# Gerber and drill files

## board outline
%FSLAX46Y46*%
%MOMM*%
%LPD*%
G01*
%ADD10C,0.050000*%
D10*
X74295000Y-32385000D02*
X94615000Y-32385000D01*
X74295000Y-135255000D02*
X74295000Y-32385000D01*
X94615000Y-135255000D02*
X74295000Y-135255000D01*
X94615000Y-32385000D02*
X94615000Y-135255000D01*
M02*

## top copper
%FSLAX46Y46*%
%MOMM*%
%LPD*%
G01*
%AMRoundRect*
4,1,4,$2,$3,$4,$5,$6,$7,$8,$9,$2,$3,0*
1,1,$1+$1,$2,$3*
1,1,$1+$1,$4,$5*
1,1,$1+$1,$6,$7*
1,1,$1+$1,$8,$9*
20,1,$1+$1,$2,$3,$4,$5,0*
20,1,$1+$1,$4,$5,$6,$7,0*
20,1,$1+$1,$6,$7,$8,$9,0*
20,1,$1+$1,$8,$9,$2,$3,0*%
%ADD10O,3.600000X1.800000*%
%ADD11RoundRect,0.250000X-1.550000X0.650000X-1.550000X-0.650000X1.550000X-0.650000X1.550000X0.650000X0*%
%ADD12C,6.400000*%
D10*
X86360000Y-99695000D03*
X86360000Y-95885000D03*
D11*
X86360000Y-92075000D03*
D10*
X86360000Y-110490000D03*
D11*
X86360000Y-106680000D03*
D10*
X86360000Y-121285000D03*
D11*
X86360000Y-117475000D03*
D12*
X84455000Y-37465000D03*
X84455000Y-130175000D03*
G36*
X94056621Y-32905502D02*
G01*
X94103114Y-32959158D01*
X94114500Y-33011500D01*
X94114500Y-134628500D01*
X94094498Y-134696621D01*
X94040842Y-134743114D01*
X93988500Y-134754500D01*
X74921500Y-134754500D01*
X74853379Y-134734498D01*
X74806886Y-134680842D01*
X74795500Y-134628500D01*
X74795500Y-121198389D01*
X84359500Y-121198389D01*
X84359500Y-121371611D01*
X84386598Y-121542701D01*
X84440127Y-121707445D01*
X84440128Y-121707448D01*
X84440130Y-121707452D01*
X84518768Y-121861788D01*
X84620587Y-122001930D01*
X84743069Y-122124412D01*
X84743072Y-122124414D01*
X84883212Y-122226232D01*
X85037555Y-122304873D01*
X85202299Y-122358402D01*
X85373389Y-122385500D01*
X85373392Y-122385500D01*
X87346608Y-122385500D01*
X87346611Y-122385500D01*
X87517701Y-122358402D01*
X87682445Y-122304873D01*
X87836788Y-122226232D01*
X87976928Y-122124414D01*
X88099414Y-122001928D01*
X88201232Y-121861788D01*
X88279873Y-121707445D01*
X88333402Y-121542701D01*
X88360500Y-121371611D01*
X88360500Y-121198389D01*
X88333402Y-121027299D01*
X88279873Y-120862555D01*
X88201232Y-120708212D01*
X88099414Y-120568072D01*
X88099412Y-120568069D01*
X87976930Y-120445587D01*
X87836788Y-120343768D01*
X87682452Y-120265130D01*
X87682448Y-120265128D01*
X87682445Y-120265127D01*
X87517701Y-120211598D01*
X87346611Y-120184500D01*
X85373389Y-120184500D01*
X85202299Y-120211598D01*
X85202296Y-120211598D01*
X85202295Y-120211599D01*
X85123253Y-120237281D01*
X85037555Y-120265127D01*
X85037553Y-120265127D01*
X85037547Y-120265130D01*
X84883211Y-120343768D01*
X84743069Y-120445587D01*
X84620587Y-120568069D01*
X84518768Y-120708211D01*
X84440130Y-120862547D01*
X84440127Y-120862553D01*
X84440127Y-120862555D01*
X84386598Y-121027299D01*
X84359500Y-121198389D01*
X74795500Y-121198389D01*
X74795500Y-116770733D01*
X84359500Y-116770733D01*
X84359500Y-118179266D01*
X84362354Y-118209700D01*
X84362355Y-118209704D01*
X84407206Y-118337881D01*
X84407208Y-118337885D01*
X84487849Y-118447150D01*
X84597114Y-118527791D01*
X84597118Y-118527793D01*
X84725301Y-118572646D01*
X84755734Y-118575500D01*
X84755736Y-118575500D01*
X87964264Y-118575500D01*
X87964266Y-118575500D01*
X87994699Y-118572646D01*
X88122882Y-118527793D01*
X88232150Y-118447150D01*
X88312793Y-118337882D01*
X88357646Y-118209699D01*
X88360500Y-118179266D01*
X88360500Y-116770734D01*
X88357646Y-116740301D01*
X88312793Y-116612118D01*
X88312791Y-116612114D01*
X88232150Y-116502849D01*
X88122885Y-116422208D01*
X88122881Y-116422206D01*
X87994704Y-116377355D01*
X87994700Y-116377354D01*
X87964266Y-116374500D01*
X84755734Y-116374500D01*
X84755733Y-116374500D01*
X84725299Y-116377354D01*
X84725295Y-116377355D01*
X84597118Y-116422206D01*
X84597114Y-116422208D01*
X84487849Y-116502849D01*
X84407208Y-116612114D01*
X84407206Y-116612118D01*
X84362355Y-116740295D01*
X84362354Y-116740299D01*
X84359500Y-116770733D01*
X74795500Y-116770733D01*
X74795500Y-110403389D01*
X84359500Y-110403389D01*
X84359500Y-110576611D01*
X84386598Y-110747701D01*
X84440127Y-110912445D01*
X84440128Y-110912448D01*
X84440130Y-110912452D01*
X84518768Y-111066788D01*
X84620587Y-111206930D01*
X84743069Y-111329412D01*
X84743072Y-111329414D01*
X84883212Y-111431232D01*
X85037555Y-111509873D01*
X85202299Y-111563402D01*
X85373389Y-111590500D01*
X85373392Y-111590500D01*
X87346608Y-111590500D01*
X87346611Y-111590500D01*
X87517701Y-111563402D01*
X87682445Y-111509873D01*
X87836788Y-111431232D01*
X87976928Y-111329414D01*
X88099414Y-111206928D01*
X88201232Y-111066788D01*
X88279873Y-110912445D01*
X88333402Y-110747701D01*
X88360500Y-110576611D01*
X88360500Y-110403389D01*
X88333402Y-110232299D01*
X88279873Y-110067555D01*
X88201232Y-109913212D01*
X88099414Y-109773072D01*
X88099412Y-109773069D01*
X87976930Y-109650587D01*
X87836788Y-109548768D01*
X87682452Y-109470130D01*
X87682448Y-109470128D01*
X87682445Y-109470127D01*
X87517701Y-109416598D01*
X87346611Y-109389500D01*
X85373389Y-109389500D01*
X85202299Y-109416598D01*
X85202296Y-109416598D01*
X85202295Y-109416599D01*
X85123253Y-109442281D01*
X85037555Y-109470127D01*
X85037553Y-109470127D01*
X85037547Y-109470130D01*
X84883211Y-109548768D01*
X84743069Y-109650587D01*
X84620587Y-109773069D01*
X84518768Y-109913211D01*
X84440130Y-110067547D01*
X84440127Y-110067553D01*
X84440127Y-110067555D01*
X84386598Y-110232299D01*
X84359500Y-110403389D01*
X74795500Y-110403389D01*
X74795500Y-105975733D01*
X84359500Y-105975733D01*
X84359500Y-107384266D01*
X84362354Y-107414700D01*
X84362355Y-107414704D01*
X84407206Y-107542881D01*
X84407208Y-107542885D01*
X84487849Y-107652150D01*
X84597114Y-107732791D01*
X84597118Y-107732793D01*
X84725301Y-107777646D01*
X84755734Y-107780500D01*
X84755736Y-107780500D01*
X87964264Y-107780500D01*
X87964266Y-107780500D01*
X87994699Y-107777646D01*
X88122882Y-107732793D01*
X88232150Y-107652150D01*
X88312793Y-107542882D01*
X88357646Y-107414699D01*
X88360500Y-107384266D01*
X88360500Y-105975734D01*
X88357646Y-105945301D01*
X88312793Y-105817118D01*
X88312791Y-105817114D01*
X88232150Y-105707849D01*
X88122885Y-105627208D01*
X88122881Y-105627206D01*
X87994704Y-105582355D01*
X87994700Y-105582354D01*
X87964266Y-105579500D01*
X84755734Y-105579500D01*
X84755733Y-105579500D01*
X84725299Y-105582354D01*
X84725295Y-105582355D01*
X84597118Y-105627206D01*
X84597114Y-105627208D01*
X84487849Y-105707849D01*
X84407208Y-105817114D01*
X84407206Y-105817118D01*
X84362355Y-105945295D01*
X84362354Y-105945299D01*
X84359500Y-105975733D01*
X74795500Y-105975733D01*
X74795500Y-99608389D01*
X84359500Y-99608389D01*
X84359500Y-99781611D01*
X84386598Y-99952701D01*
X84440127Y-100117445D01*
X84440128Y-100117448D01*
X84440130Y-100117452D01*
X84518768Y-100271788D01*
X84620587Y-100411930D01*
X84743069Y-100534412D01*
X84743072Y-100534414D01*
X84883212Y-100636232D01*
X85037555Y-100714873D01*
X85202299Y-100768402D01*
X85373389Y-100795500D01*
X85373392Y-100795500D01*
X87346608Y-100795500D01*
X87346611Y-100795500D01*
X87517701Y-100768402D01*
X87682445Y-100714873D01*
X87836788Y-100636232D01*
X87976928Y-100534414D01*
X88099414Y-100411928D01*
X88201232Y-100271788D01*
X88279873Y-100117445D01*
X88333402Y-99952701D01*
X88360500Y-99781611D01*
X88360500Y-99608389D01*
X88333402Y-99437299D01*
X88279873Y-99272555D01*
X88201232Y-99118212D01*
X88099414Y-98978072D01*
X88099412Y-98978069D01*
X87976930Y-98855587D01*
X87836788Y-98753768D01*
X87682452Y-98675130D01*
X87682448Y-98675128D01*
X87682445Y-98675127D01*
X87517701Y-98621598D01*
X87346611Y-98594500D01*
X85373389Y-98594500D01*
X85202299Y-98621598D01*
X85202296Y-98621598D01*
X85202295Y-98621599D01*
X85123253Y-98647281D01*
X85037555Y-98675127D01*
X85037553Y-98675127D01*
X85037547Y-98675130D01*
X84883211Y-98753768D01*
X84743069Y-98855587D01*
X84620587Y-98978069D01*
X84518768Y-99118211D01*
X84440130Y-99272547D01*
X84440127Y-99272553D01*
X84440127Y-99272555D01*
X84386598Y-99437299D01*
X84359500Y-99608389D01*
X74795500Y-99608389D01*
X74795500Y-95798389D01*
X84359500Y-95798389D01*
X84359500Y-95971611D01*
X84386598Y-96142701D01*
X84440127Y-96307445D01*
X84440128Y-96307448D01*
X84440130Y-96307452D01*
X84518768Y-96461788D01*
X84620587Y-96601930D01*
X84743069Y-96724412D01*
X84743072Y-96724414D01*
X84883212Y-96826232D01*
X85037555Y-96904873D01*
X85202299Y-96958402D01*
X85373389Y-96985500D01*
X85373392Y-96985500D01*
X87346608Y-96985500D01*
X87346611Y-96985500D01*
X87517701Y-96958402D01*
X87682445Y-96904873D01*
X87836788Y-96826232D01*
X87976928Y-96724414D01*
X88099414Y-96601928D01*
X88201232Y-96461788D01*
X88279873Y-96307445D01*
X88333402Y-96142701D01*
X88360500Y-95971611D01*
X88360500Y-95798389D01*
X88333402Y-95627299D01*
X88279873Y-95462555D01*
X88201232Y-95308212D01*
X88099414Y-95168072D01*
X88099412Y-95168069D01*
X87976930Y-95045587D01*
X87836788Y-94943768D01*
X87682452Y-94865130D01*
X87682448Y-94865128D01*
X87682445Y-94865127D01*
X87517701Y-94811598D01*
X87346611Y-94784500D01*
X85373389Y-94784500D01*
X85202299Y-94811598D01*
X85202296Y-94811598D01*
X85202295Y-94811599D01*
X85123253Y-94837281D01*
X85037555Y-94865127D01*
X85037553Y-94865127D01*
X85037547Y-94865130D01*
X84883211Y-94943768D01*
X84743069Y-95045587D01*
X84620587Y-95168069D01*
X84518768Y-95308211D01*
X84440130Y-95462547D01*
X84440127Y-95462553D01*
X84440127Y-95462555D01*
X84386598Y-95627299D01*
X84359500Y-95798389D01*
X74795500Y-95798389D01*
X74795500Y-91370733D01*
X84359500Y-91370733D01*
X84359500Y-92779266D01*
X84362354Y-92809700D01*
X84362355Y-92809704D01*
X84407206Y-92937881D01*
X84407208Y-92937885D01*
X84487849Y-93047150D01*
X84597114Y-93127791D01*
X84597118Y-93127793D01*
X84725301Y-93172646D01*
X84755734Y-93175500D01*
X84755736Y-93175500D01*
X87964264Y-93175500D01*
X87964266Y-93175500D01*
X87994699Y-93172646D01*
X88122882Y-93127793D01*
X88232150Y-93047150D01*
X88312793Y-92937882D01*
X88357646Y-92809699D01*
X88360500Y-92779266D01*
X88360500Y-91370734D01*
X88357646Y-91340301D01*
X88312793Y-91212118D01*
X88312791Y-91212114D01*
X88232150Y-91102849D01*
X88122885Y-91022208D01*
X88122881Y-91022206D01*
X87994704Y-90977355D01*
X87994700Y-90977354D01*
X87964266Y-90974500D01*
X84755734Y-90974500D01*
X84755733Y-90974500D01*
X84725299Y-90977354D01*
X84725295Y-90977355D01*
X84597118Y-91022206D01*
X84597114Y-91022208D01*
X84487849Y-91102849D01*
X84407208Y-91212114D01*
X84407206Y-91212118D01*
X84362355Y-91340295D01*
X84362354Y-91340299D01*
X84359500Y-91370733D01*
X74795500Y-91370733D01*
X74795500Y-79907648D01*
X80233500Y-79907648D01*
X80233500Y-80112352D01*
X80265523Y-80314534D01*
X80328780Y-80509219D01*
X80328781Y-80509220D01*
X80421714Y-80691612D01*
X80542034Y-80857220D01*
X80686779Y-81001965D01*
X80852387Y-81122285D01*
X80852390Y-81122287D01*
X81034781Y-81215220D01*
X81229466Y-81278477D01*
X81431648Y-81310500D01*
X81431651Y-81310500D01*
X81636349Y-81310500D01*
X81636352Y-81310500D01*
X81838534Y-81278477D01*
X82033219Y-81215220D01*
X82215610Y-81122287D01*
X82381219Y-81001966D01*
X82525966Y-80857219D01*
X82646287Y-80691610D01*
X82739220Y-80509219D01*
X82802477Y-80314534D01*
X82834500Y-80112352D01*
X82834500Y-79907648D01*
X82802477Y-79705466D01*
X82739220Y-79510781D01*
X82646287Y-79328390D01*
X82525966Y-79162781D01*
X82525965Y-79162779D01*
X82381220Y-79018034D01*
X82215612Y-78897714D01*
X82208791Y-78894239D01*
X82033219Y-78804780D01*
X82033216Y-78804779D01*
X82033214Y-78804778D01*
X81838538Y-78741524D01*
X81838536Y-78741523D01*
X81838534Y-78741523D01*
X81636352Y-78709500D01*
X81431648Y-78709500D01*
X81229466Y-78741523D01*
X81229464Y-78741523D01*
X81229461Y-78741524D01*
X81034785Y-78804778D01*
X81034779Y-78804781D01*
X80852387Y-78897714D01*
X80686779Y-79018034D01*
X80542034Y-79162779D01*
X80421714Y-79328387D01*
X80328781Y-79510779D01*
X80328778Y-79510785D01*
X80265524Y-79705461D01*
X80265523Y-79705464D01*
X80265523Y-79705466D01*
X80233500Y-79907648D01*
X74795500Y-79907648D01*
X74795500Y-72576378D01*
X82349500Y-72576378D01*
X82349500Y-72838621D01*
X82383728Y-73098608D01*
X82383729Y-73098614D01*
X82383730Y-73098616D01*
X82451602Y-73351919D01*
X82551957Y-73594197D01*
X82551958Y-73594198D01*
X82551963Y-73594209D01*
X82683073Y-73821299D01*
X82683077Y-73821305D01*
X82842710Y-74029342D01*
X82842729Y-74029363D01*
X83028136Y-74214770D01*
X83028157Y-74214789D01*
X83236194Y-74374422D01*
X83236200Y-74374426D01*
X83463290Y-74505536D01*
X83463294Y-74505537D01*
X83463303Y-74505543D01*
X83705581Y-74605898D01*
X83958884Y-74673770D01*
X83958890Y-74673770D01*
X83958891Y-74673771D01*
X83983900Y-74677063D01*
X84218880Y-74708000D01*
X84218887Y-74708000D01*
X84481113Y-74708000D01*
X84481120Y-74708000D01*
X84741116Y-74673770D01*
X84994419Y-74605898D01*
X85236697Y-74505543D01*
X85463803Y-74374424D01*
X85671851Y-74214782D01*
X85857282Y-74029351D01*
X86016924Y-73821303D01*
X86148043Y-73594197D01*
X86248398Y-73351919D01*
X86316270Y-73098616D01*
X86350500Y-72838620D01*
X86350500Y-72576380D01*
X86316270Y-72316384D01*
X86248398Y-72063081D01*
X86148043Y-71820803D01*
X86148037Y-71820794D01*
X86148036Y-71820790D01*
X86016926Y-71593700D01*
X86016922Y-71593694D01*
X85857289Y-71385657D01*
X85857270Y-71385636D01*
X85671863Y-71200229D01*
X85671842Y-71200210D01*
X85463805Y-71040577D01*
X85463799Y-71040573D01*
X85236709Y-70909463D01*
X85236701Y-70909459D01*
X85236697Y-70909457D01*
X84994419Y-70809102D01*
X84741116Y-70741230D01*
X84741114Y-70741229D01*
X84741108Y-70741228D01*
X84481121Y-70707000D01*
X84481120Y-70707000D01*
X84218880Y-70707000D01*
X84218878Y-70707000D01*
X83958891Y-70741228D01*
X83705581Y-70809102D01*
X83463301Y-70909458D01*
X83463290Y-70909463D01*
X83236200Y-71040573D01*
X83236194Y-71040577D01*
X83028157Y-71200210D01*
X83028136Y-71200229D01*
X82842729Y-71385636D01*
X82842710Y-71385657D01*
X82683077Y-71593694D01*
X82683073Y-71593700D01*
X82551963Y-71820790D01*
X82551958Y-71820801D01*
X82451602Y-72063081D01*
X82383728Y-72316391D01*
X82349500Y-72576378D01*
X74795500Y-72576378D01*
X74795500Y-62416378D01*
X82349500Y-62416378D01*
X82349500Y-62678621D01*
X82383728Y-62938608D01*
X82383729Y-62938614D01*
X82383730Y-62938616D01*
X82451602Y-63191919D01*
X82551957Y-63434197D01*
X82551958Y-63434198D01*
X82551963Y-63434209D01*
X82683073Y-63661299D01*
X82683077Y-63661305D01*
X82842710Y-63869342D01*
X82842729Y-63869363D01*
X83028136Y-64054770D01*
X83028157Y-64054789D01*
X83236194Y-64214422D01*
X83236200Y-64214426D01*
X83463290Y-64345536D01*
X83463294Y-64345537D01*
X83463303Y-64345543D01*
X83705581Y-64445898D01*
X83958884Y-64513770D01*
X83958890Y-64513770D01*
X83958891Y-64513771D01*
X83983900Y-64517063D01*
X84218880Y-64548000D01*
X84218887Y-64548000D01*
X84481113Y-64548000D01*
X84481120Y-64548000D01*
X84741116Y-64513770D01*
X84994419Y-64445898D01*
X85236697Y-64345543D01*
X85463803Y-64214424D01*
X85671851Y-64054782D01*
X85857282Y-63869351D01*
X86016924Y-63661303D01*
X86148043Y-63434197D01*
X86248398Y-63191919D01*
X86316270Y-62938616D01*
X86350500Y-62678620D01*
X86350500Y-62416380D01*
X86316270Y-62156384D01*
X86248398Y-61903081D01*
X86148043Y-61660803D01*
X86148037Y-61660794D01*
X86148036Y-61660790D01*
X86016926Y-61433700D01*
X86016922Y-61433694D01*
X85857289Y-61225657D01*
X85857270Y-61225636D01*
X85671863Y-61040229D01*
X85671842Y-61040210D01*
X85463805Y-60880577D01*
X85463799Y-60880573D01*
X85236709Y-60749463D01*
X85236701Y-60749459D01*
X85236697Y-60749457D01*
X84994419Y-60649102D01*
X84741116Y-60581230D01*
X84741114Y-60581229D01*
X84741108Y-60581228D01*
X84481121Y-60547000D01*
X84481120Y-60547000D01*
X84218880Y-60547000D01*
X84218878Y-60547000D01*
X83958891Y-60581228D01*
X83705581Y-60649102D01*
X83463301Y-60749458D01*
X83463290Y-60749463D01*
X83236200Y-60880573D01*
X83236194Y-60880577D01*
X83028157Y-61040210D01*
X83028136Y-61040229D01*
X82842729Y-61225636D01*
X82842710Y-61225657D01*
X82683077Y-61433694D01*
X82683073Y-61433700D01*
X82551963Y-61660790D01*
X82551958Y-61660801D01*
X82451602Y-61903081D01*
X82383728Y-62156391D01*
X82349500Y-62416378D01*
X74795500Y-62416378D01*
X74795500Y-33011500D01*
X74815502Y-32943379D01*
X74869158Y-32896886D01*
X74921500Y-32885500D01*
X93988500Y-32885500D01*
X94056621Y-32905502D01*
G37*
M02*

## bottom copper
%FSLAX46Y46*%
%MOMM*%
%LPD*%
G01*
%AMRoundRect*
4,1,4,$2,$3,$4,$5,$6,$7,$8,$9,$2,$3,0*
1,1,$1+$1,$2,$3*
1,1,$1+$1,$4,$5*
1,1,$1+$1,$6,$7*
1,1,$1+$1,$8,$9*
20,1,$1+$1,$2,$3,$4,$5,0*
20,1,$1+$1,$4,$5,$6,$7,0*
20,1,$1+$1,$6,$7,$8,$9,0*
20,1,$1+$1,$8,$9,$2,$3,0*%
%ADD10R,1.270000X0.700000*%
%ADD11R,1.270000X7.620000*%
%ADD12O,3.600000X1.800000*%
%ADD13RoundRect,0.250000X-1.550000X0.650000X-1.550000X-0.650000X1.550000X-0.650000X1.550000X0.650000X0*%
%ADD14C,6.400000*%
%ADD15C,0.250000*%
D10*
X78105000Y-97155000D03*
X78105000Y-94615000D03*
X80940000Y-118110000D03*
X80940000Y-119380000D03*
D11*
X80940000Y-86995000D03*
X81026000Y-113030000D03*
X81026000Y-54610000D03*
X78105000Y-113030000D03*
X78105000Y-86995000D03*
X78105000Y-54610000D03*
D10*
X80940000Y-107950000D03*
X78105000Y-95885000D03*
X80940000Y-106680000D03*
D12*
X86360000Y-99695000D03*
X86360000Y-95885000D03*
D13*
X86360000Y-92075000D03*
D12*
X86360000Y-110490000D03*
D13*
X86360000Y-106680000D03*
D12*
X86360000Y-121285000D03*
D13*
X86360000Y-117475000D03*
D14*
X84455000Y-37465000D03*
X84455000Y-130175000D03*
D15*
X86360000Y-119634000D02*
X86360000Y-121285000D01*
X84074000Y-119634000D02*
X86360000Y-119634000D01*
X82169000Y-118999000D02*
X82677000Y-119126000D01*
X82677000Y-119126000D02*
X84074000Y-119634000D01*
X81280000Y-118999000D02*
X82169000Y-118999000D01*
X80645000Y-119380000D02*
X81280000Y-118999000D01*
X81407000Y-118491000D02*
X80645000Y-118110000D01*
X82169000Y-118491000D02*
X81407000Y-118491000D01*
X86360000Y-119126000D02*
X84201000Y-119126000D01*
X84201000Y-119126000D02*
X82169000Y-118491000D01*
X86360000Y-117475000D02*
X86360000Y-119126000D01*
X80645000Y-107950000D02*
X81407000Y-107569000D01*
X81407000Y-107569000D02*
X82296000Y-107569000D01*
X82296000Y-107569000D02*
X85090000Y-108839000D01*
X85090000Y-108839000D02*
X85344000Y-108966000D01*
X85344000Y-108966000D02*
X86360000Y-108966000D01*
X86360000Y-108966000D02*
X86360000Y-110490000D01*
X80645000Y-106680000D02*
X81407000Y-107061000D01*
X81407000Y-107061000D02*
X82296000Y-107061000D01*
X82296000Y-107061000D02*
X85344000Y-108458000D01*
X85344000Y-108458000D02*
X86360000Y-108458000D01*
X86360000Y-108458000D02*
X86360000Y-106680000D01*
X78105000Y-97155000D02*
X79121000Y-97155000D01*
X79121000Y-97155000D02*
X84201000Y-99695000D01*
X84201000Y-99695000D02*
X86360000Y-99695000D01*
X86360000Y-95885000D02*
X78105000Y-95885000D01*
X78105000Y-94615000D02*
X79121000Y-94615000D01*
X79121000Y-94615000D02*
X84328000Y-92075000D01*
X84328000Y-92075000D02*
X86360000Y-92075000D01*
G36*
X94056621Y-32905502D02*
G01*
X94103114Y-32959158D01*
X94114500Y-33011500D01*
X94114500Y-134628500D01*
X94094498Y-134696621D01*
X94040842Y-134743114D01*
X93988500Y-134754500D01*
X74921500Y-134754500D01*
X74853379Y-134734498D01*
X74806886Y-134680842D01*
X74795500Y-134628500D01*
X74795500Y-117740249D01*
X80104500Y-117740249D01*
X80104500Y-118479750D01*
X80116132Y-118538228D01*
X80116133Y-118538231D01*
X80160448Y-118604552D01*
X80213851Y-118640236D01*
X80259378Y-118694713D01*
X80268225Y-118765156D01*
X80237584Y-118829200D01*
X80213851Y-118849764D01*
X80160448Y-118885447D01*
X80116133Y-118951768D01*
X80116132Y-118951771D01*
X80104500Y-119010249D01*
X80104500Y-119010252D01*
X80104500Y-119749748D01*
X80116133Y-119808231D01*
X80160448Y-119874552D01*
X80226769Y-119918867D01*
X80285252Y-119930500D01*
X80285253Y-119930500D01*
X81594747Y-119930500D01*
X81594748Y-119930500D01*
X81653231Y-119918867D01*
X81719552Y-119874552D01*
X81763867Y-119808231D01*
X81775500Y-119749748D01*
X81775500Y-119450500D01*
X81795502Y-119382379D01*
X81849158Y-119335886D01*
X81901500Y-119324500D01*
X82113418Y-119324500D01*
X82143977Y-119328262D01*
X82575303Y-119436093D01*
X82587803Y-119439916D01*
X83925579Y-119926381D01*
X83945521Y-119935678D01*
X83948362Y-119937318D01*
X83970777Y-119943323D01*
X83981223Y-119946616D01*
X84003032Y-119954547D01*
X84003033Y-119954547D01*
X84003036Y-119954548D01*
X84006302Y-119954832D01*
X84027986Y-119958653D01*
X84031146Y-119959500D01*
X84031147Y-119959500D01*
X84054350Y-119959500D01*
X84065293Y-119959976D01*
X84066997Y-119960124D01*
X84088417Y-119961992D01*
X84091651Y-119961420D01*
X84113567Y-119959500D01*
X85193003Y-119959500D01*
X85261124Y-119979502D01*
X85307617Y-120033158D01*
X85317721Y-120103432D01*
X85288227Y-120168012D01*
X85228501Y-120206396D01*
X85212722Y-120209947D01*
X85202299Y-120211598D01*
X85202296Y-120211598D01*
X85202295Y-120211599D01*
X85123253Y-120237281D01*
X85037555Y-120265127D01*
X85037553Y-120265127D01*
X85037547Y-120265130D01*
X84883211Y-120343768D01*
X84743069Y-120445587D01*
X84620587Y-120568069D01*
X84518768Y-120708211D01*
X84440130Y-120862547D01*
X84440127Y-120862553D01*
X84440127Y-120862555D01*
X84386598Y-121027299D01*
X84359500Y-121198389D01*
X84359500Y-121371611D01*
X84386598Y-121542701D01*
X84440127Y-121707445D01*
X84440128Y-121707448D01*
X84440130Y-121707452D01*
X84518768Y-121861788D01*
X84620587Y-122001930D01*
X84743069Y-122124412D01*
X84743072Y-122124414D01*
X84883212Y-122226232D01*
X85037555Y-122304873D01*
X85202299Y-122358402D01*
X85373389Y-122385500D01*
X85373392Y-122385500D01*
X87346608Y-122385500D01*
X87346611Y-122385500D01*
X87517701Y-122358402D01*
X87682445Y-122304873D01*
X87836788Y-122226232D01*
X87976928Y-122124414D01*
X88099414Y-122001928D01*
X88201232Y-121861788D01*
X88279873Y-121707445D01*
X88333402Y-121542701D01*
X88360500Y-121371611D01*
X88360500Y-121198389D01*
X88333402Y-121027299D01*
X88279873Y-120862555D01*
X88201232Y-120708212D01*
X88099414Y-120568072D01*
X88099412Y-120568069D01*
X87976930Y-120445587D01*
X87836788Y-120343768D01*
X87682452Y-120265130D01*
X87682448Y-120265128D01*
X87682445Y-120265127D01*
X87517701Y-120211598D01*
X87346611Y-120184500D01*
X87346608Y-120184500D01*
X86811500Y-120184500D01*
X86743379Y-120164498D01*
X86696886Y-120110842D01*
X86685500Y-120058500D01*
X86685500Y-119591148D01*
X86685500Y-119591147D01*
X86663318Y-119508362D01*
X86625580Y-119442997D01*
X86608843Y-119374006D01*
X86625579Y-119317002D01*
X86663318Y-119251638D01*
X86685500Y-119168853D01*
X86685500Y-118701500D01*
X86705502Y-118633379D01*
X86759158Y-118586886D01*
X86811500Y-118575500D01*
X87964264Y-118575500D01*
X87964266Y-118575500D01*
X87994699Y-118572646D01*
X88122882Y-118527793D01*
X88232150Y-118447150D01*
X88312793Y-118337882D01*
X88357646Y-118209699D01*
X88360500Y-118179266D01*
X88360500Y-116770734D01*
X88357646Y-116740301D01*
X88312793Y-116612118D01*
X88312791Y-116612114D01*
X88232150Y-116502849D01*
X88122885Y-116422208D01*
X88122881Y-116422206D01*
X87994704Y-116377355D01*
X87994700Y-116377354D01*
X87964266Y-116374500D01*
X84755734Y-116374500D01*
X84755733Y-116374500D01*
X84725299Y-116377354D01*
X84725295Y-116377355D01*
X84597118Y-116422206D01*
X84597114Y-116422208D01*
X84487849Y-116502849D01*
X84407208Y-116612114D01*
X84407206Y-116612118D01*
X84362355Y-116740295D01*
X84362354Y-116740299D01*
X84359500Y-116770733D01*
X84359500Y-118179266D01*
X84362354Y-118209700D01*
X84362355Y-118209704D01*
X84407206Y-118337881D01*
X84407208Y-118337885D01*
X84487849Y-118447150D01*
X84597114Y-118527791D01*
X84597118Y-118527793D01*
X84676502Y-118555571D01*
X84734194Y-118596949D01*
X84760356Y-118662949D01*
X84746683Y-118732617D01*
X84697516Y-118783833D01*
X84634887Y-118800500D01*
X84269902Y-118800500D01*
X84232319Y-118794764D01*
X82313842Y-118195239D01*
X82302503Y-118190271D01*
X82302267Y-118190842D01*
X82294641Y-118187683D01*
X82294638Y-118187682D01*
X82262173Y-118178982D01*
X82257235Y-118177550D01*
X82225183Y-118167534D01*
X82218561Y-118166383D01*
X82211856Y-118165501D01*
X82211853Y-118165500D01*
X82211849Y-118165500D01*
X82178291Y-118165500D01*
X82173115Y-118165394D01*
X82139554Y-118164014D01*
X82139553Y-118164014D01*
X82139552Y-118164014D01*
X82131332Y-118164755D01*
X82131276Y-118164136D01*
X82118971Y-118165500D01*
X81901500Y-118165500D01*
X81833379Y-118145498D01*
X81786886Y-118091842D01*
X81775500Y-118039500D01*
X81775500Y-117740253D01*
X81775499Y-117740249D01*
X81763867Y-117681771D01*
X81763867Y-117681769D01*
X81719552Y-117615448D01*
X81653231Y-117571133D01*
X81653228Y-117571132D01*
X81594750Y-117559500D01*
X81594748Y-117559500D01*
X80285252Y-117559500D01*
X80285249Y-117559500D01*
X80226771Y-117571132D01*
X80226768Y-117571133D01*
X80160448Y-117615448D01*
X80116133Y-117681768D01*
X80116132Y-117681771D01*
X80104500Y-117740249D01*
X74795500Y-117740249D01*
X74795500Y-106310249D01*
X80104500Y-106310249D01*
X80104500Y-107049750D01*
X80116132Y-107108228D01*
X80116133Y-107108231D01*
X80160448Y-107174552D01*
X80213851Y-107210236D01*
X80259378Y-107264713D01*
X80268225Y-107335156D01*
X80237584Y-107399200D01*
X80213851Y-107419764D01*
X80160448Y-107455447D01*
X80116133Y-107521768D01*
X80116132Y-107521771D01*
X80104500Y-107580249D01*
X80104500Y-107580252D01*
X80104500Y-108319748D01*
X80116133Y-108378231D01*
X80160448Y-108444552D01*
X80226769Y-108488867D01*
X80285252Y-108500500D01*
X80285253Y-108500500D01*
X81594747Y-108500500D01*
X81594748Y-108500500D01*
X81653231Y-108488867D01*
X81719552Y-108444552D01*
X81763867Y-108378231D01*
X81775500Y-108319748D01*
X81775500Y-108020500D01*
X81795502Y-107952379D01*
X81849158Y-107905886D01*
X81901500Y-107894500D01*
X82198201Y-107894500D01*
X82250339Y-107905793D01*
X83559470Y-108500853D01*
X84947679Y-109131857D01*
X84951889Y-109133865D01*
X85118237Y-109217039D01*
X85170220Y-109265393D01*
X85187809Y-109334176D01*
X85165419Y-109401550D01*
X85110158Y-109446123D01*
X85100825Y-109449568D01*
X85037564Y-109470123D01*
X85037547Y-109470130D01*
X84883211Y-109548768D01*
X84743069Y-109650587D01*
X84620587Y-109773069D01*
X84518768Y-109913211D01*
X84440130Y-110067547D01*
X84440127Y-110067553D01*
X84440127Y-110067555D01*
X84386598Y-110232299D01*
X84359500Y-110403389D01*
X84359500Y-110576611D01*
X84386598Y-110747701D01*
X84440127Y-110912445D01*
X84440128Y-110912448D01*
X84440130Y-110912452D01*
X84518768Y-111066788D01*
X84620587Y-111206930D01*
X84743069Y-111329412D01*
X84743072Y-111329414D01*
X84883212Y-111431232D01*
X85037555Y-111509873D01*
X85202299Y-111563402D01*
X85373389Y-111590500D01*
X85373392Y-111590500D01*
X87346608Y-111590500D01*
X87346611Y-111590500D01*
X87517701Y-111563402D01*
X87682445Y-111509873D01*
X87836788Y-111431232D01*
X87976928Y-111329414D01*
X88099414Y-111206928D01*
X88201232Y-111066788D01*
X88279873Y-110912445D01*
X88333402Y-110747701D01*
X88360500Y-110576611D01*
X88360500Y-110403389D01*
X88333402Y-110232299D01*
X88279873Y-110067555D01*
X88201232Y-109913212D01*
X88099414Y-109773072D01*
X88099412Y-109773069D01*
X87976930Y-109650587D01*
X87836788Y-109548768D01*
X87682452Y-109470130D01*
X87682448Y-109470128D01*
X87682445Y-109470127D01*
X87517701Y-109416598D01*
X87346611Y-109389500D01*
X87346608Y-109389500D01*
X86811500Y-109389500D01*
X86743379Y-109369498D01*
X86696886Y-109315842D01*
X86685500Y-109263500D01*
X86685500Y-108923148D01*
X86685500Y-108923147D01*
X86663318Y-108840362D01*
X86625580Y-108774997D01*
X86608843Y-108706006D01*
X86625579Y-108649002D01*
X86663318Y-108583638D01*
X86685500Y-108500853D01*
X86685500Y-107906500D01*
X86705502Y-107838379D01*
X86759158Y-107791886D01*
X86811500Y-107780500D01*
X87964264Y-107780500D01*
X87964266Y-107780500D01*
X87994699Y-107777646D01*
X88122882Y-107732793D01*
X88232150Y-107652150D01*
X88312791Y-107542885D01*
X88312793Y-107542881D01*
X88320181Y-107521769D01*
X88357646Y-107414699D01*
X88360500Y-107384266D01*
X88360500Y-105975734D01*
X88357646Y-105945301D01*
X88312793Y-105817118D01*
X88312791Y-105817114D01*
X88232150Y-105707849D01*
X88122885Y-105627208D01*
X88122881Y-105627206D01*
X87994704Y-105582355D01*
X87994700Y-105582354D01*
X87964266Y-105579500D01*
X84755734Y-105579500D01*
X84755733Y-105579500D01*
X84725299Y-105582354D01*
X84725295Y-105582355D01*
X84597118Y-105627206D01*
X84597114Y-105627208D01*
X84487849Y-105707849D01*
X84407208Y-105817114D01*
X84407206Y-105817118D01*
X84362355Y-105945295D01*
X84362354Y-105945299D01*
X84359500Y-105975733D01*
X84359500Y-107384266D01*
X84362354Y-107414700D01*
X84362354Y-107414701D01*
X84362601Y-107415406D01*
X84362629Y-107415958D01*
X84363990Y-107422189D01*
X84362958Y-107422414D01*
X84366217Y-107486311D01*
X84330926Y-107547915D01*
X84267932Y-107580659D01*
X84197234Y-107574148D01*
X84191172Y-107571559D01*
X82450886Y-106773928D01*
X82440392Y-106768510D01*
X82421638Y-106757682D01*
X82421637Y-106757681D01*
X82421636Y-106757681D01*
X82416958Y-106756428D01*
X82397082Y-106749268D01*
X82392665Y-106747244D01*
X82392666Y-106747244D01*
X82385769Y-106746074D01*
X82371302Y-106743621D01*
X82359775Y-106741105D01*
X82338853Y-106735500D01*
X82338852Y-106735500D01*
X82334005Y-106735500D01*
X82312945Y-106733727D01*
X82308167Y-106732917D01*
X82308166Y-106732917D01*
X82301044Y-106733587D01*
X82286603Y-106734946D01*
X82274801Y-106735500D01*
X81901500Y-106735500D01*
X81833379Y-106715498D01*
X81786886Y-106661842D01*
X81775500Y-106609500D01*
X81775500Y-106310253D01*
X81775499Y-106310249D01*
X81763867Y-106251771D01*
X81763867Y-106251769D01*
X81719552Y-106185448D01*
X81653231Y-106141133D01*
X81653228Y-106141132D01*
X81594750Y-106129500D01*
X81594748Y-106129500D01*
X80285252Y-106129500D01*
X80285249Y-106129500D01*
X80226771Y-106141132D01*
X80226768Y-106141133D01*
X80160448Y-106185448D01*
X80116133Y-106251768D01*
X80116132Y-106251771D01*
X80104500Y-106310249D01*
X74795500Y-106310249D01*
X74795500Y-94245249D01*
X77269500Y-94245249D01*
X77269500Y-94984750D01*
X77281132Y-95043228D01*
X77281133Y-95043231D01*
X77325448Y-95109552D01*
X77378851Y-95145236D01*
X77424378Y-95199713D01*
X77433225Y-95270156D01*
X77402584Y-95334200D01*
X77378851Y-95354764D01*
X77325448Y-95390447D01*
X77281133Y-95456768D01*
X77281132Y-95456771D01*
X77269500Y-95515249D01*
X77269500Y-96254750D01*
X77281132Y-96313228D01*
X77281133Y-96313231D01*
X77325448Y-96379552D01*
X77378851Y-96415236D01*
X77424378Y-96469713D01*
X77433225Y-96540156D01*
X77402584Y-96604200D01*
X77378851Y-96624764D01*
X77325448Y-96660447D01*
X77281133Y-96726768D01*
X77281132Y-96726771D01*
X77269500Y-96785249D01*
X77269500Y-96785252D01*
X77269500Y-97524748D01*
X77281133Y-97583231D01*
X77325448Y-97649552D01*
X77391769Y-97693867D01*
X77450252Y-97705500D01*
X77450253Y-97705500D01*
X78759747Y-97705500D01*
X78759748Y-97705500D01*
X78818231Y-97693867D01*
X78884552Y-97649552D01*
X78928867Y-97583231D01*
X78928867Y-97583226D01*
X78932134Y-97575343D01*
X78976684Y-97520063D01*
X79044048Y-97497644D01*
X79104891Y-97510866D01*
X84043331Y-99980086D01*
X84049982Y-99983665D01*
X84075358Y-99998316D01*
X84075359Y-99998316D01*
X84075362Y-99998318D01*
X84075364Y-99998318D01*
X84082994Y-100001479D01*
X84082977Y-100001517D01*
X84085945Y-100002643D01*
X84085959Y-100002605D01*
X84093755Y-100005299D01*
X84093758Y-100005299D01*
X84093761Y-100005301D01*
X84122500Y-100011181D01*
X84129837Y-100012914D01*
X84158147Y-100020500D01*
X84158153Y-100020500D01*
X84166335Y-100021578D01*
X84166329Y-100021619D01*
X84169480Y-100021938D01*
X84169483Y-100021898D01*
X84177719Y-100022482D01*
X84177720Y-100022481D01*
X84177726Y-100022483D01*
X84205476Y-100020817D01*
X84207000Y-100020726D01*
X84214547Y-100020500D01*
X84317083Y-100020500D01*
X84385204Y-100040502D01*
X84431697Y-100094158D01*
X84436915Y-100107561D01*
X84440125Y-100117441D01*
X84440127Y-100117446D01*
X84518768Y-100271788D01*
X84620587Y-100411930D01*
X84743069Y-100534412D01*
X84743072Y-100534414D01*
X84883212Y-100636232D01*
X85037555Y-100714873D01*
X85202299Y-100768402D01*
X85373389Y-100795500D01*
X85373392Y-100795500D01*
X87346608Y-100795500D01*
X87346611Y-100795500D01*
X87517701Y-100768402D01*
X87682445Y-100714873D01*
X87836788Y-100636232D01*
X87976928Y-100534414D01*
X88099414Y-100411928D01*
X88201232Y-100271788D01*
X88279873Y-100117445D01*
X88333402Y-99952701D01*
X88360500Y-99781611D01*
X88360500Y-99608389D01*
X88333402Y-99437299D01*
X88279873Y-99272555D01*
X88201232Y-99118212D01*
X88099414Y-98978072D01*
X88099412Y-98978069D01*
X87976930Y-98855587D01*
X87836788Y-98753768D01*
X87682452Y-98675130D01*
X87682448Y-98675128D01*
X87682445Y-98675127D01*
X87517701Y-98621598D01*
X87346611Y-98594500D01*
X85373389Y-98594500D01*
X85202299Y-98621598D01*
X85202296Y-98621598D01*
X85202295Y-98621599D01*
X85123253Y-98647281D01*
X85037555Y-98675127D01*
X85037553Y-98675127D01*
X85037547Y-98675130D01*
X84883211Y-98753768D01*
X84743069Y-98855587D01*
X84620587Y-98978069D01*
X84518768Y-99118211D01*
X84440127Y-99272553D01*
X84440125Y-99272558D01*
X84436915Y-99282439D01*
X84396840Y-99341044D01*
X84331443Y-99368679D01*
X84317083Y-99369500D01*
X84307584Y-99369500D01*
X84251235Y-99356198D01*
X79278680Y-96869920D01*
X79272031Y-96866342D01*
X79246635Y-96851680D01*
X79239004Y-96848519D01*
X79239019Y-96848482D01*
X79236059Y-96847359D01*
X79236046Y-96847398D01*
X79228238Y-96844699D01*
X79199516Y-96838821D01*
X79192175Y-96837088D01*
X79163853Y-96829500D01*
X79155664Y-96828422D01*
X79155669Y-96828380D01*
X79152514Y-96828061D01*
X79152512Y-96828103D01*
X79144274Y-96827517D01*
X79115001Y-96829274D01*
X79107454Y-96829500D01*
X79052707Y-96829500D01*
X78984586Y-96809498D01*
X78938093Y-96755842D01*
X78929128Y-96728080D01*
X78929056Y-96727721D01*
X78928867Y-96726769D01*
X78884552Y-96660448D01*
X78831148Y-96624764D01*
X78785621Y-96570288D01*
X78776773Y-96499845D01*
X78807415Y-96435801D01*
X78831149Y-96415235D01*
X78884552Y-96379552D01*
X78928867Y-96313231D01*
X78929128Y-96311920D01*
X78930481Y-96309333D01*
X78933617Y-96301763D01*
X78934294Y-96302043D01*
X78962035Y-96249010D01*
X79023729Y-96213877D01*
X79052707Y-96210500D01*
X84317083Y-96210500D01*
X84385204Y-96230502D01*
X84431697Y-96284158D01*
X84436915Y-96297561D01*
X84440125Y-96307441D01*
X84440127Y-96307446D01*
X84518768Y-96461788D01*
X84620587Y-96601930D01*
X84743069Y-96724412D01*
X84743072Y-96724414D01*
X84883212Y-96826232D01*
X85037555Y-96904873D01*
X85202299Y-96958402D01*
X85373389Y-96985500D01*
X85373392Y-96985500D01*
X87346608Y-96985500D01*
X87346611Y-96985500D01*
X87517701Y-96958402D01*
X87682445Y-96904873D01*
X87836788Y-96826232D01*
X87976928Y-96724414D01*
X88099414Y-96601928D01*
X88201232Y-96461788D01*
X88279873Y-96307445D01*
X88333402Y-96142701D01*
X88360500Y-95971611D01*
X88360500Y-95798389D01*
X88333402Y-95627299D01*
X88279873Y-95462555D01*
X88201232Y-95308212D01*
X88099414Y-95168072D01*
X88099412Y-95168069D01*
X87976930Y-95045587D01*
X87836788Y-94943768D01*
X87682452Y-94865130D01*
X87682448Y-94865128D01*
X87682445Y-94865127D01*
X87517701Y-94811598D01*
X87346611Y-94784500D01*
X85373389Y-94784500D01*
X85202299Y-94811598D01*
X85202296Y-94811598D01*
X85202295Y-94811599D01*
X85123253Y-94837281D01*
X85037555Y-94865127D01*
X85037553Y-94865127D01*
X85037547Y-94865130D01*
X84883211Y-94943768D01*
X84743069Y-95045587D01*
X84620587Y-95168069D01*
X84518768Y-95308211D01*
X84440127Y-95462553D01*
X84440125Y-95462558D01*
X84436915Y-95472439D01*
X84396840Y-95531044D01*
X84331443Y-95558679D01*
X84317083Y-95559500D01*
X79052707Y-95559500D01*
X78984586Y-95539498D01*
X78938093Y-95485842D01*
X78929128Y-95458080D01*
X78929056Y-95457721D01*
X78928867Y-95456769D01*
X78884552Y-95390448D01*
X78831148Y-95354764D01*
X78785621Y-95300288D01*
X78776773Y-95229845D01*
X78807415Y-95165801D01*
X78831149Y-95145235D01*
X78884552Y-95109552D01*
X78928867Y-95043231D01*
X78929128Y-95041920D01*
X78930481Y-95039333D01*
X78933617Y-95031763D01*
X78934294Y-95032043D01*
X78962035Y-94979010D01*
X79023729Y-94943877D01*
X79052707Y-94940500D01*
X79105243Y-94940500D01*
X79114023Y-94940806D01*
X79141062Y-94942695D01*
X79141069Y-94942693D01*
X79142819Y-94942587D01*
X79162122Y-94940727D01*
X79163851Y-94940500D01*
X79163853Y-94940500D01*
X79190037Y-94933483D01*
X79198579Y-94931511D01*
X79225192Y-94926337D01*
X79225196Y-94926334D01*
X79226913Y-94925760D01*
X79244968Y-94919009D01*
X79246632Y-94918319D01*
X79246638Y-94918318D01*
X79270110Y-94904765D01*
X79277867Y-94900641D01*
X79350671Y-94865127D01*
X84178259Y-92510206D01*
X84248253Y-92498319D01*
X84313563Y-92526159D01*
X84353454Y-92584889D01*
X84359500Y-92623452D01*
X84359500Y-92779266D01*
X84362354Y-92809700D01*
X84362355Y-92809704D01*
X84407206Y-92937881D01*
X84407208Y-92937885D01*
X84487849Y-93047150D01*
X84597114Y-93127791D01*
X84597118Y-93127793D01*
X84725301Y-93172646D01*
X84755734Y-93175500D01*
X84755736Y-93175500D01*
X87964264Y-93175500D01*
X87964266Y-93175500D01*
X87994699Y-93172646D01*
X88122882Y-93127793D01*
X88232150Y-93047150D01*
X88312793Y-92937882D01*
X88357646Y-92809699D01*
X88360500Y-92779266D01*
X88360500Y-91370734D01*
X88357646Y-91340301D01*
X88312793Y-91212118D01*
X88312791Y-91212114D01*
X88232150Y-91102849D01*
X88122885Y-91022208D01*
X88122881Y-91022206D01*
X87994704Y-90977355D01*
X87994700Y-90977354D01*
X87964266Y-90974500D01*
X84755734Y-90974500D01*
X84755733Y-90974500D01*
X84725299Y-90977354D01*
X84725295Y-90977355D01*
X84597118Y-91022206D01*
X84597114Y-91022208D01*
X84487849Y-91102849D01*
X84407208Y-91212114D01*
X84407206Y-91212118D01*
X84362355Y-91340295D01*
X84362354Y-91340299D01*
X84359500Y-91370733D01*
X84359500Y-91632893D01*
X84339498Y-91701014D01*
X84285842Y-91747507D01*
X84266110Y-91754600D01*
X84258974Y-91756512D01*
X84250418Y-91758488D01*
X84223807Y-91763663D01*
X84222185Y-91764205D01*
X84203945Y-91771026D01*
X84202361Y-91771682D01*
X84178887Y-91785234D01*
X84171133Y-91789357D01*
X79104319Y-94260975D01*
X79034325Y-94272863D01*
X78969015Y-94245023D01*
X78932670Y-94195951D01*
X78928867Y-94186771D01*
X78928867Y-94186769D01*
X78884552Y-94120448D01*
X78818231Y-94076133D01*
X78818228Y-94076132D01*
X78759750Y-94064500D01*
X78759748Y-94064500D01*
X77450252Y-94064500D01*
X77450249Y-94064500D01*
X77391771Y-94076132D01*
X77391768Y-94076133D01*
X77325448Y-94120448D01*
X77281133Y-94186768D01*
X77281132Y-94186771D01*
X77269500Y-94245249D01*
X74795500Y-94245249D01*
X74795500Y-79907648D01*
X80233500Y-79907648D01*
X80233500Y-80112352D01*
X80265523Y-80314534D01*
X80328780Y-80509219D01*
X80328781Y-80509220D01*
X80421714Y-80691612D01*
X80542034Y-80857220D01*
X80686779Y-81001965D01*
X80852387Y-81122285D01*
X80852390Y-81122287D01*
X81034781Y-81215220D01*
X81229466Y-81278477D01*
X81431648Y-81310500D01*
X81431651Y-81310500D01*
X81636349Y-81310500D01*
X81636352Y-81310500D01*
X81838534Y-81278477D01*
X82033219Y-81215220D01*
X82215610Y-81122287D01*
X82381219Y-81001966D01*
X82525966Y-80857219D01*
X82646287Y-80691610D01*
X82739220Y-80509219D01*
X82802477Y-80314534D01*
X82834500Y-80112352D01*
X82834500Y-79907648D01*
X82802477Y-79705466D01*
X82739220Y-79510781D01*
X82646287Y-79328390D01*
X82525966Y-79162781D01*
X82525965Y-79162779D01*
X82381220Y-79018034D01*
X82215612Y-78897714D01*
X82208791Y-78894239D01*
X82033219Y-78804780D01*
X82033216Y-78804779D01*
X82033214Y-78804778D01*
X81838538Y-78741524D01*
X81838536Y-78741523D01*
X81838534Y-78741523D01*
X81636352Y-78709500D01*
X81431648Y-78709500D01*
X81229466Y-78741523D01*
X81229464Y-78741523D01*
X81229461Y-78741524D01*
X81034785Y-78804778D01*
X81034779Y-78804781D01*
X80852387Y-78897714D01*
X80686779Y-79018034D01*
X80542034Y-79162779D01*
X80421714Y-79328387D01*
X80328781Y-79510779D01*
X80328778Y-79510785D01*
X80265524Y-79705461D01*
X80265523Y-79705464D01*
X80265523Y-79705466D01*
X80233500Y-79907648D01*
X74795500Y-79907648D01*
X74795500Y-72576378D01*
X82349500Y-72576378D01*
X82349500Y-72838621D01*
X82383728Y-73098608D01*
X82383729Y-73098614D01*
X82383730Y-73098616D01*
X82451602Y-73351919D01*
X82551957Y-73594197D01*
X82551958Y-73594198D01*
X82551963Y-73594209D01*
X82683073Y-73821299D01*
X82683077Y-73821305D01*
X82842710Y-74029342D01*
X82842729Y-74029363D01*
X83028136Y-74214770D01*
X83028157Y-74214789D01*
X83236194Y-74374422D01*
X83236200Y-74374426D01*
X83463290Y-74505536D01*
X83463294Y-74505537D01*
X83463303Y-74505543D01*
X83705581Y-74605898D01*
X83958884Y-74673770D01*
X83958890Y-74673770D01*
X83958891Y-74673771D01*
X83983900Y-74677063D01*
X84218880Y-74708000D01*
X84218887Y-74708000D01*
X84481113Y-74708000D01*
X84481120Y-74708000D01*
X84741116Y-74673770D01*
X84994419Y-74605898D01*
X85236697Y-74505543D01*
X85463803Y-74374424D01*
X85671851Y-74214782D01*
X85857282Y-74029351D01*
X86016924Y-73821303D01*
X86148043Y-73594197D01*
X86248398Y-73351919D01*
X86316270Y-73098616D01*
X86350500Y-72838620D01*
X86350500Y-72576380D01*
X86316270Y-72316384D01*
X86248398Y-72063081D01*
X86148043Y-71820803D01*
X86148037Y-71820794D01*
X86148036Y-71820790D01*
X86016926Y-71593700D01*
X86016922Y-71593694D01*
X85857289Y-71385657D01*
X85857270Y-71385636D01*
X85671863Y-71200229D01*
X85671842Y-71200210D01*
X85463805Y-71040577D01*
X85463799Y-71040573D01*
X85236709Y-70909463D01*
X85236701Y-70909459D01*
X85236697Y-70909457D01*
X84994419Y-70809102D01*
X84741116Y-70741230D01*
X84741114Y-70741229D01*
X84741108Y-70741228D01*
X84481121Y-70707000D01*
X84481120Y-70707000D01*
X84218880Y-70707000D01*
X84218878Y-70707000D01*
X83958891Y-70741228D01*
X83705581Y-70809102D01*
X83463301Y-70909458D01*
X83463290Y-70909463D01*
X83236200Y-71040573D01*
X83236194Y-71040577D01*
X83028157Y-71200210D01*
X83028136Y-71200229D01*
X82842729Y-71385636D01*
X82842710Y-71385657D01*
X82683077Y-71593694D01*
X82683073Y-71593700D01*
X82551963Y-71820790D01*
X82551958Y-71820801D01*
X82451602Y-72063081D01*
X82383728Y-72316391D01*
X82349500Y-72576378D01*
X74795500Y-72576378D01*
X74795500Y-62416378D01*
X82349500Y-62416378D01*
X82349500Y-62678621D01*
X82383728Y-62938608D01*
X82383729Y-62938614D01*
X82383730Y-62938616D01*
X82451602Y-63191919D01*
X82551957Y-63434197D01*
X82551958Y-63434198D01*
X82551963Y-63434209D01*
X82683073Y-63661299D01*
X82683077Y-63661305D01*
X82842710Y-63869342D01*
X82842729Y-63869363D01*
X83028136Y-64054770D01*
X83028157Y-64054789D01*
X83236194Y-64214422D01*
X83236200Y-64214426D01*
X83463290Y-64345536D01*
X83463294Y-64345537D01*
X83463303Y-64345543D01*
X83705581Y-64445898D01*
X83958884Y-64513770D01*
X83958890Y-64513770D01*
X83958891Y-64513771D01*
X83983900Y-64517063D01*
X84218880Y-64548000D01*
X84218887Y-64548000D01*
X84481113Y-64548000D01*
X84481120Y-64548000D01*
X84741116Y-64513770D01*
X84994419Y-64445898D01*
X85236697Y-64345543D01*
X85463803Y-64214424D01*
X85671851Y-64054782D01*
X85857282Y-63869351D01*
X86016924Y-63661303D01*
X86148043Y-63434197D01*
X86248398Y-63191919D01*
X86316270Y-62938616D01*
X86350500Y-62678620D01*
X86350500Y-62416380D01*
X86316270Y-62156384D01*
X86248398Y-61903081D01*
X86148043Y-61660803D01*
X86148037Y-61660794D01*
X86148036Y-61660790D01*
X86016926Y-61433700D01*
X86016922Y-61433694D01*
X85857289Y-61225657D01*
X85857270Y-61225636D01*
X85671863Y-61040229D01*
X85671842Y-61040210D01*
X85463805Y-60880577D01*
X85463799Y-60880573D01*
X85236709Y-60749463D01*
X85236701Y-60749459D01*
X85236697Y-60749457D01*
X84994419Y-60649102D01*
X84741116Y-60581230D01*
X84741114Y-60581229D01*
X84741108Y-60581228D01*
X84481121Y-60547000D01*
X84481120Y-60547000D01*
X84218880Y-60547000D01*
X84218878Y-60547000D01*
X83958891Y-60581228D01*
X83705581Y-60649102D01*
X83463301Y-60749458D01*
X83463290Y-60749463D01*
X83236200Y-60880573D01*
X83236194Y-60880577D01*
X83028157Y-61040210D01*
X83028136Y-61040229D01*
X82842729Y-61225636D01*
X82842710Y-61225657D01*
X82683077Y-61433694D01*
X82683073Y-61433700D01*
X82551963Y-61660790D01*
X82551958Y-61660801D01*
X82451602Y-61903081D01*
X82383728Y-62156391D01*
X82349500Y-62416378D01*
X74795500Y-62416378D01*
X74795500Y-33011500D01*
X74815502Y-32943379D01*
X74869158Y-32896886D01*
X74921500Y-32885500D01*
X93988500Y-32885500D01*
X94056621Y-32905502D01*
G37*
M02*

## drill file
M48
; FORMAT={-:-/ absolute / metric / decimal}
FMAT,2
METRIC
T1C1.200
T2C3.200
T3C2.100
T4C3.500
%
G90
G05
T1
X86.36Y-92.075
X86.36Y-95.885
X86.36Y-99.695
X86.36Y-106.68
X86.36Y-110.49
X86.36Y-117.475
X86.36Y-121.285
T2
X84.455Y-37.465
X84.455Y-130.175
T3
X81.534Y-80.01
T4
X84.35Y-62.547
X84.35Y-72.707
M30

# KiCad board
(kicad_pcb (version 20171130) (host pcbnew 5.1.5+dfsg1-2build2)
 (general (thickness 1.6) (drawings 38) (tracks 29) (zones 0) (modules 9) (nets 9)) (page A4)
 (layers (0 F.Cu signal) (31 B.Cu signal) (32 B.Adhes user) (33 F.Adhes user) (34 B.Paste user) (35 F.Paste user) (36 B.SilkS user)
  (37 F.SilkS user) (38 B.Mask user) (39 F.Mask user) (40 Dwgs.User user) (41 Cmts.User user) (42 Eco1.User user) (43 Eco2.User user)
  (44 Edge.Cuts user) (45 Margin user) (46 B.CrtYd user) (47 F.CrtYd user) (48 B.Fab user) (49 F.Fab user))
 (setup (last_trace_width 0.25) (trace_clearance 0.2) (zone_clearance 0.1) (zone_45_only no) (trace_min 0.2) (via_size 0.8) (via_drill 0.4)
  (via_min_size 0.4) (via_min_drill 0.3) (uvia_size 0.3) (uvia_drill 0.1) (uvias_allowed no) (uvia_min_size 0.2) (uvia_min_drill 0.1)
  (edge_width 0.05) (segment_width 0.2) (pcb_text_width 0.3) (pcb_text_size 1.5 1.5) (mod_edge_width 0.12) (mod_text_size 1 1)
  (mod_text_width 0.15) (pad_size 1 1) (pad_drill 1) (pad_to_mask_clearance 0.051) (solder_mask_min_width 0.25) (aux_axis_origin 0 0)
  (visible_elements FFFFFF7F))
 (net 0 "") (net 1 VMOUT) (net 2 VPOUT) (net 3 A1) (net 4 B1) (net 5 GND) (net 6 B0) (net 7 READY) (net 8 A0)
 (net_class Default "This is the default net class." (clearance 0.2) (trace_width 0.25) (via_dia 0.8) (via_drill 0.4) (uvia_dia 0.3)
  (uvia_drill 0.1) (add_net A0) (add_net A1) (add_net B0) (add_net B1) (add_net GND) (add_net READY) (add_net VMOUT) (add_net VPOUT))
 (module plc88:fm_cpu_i (layer F.Cu) (at 80.645 55.245)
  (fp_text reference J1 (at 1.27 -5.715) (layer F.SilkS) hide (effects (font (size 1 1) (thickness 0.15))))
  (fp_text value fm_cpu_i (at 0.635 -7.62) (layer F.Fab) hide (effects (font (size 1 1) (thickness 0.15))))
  (pad 3 smd rect (at -2.54 41.91) (size 1.27 0.7) (layers B.Cu B.Paste B.Mask) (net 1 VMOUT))
  (pad 1 smd rect (at -2.54 39.37) (size 1.27 0.7) (layers B.Cu B.Paste B.Mask) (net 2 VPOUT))
  (pad 6 smd rect (at 0.295 62.865) (size 1.27 0.7) (layers B.Cu B.Paste B.Mask) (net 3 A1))
  (pad 7 smd rect (at 0.295 64.135) (size 1.27 0.7) (layers B.Cu B.Paste B.Mask) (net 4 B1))
  (pad 8 smd rect (at 0.295 31.75) (size 1.27 7.62) (layers B.Cu B.Paste B.Mask) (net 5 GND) (zone_connect 2))
  (pad 8 smd rect (at 0.381 57.785) (size 1.27 7.62) (layers B.Cu B.Paste B.Mask) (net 5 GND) (zone_connect 2))
  (pad 8 smd rect (at 0.381 -0.635) (size 1.27 7.62) (layers B.Cu B.Paste B.Mask) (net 5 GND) (zone_connect 2))
  (pad 8 smd rect (at -2.54 57.785) (size 1.27 7.62) (layers B.Cu B.Paste B.Mask) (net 5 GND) (zone_connect 2))
  (pad 8 smd rect (at -2.54 31.75) (size 1.27 7.62) (layers B.Cu B.Paste B.Mask) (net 5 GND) (zone_connect 2))
  (pad 8 smd rect (at -2.54 -0.635) (size 1.27 7.62) (layers B.Cu B.Paste B.Mask) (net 5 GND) (zone_connect 2))
  (pad 5 smd rect (at 0.295 52.705) (size 1.27 0.7) (layers B.Cu B.Paste B.Mask) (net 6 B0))
  (pad 2 smd rect (at -2.54 40.64) (size 1.27 0.7) (layers B.Cu B.Paste B.Mask) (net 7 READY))
  (pad 4 smd rect (at 0.295 51.435) (size 1.27 0.7) (layers B.Cu B.Paste B.Mask) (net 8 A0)))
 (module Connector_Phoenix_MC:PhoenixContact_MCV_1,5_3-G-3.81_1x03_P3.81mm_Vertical (layer F.Cu) (at 86.36 92.075 270)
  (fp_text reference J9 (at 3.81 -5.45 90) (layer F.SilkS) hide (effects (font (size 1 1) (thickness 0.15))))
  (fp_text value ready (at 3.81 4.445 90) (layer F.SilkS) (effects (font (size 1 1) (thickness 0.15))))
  (pad 3 thru_hole oval (at 7.62 0 270) (size 1.8 3.6) (drill 1.2) (layers *.Cu *.Mask) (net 1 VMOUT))
  (pad 2 thru_hole oval (at 3.81 0 270) (size 1.8 3.6) (drill 1.2) (layers *.Cu *.Mask) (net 7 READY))
  (pad 1 thru_hole roundrect (at 0 0 270) (size 1.8 3.6) (drill 1.2) (layers *.Cu *.Mask) (roundrect_rratio 0.138889) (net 2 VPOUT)))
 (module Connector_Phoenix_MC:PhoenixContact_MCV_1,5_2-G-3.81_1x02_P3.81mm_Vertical (layer F.Cu) (at 86.36 106.68 270)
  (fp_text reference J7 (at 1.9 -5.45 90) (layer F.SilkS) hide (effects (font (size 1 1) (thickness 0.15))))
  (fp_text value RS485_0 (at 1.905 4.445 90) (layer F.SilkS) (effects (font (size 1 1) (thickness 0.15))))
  (pad 2 thru_hole oval (at 3.81 0 270) (size 1.8 3.6) (drill 1.2) (layers *.Cu *.Mask) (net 6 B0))
  (pad 1 thru_hole roundrect (at 0 0 270) (size 1.8 3.6) (drill 1.2) (layers *.Cu *.Mask) (roundrect_rratio 0.138889) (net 8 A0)))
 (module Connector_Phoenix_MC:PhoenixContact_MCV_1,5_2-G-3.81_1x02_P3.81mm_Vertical (layer F.Cu) (at 86.36 117.475 270)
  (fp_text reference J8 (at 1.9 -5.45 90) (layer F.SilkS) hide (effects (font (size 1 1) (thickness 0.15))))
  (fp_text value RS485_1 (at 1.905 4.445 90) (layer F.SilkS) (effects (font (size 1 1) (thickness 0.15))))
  (pad 2 thru_hole oval (at 3.81 0 270) (size 1.8 3.6) (drill 1.2) (layers *.Cu *.Mask) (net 4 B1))
  (pad 1 thru_hole roundrect (at 0 0 270) (size 1.8 3.6) (drill 1.2) (layers *.Cu *.Mask) (roundrect_rratio 0.138889) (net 3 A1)))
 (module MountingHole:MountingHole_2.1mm (layer F.Cu) (at 81.534 80.01)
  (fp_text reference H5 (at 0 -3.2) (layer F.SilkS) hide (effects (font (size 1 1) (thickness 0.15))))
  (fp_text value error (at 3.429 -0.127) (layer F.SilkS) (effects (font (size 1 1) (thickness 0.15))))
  (pad "" np_thru_hole circle (at 0 0) (size 2.1 2.1) (drill 2.1) (layers *.Cu *.Mask)))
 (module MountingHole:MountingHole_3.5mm (layer F.Cu) (at 84.35 72.7075)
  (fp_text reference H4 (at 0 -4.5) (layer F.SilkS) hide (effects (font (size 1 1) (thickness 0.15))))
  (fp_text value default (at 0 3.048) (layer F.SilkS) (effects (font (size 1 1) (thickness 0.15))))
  (pad 1 np_thru_hole circle (at 0 0) (size 3.5 3.5) (drill 3.5) (layers *.Cu *.Mask)))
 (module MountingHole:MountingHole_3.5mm (layer F.Cu) (at 84.35 62.5475)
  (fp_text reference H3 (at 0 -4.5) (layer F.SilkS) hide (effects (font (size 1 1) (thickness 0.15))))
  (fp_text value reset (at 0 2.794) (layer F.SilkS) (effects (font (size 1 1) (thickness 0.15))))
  (pad 1 np_thru_hole circle (at 0 0) (size 3.5 3.5) (drill 3.5) (layers *.Cu *.Mask)))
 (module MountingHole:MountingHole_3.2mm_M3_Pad (layer F.Cu) (at 84.455 37.465)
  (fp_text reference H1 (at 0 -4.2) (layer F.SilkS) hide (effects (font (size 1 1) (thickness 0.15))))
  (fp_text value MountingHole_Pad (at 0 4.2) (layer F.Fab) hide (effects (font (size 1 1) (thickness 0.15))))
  (pad 1 thru_hole circle (at 0 0) (size 6.4 6.4) (drill 3.2) (layers *.Cu *.Mask) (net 5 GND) (zone_connect 2)))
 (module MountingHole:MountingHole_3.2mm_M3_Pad (layer F.Cu) (at 84.455 130.175)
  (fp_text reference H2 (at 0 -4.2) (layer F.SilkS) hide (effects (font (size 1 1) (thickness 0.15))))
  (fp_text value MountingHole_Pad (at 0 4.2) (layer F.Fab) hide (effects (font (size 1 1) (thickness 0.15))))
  (pad 1 thru_hole circle (at 0 0) (size 6.4 6.4) (drill 3.2) (layers *.Cu *.Mask) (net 5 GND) (zone_connect 2)))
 (gr_line (start 74.295 32.385) (end 94.615 32.385) (layer Edge.Cuts) (width 0.05))
 (gr_line (start 74.295 135.255) (end 74.295 32.385) (layer Edge.Cuts) (width 0.05))
 (gr_line (start 94.615 135.255) (end 74.295 135.255) (layer Edge.Cuts) (width 0.05))
 (gr_line (start 94.615 32.385) (end 94.615 135.255) (layer Edge.Cuts) (width 0.05))
 (segment (start 86.36 119.634) (end 86.36 121.285) (width 0.25) (layer B.Cu) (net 4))
 (segment (start 84.074 119.634) (end 86.36 119.634) (width 0.25) (layer B.Cu) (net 4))
 (segment (start 82.169 118.999) (end 82.677 119.126) (width 0.25) (layer B.Cu) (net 4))
 (segment (start 82.677 119.126) (end 84.074 119.634) (width 0.25) (layer B.Cu) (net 4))
 (segment (start 81.28 118.999) (end 82.169 118.999) (width 0.25) (layer B.Cu) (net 4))
 (segment (start 80.645 119.38) (end 81.28 118.999) (width 0.25) (layer B.Cu) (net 4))
 (segment (start 81.407 118.491) (end 80.645 118.11) (width 0.25) (layer B.Cu) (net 3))
 (segment (start 82.169 118.491) (end 81.407 118.491) (width 0.25) (layer B.Cu) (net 3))
 (segment (start 86.36 119.126) (end 84.201 119.126) (width 0.25) (layer B.Cu) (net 3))
 (segment (start 84.201 119.126) (end 82.169 118.491) (width 0.25) (layer B.Cu) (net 3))
 (segment (start 86.36 117.475) (end 86.36 119.126) (width 0.25) (layer B.Cu) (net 3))
 (segment (start 80.645 107.95) (end 81.407 107.569) (width 0.25) (layer B.Cu) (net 6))
 (segment (start 81.407 107.569) (end 82.296 107.569) (width 0.25) (layer B.Cu) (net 6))
 (segment (start 82.296 107.569) (end 85.09 108.839) (width 0.25) (layer B.Cu) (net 6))
 (segment (start 85.09 108.839) (end 85.344 108.966) (width 0.25) (layer B.Cu) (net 6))
 (segment (start 85.344 108.966) (end 86.36 108.966) (width 0.25) (layer B.Cu) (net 6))
 (segment (start 86.36 108.966) (end 86.36 110.49) (width 0.25) (layer B.Cu) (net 6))
 (segment (start 80.645 106.68) (end 81.407 107.061) (width 0.25) (layer B.Cu) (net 8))
 (segment (start 81.407 107.061) (end 82.296 107.061) (width 0.25) (layer B.Cu) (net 8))
 (segment (start 82.296 107.061) (end 85.344 108.458) (width 0.25) (layer B.Cu) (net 8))
 (segment (start 85.344 108.458) (end 86.36 108.458) (width 0.25) (layer B.Cu) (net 8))
 (segment (start 86.36 108.458) (end 86.36 106.68) (width 0.25) (layer B.Cu) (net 8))
 (segment (start 78.105 97.155) (end 79.121 97.155) (width 0.25) (layer B.Cu) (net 1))
 (segment (start 79.121 97.155) (end 84.201 99.695) (width 0.25) (layer B.Cu) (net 1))
 (segment (start 84.201 99.695) (end 86.36 99.695) (width 0.25) (layer B.Cu) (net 1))
 (segment (start 86.36 95.885) (end 78.105 95.885) (width 0.25) (layer B.Cu) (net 7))
 (segment (start 78.105 94.615) (end 79.121 94.615) (width 0.25) (layer B.Cu) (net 2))
 (segment (start 79.121 94.615) (end 84.328 92.075) (width 0.25) (layer B.Cu) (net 2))
 (segment (start 84.328 92.075) (end 86.36 92.075) (width 0.25) (layer B.Cu) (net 2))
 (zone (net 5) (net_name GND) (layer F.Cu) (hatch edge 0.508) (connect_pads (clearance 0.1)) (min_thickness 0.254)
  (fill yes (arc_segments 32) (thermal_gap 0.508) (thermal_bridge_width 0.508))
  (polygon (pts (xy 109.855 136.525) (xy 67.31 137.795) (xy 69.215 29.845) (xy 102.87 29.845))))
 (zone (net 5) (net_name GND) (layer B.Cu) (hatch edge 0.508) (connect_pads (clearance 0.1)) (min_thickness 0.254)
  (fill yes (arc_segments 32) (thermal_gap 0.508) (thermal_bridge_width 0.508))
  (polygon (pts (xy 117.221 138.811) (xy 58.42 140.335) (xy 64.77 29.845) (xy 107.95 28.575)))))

